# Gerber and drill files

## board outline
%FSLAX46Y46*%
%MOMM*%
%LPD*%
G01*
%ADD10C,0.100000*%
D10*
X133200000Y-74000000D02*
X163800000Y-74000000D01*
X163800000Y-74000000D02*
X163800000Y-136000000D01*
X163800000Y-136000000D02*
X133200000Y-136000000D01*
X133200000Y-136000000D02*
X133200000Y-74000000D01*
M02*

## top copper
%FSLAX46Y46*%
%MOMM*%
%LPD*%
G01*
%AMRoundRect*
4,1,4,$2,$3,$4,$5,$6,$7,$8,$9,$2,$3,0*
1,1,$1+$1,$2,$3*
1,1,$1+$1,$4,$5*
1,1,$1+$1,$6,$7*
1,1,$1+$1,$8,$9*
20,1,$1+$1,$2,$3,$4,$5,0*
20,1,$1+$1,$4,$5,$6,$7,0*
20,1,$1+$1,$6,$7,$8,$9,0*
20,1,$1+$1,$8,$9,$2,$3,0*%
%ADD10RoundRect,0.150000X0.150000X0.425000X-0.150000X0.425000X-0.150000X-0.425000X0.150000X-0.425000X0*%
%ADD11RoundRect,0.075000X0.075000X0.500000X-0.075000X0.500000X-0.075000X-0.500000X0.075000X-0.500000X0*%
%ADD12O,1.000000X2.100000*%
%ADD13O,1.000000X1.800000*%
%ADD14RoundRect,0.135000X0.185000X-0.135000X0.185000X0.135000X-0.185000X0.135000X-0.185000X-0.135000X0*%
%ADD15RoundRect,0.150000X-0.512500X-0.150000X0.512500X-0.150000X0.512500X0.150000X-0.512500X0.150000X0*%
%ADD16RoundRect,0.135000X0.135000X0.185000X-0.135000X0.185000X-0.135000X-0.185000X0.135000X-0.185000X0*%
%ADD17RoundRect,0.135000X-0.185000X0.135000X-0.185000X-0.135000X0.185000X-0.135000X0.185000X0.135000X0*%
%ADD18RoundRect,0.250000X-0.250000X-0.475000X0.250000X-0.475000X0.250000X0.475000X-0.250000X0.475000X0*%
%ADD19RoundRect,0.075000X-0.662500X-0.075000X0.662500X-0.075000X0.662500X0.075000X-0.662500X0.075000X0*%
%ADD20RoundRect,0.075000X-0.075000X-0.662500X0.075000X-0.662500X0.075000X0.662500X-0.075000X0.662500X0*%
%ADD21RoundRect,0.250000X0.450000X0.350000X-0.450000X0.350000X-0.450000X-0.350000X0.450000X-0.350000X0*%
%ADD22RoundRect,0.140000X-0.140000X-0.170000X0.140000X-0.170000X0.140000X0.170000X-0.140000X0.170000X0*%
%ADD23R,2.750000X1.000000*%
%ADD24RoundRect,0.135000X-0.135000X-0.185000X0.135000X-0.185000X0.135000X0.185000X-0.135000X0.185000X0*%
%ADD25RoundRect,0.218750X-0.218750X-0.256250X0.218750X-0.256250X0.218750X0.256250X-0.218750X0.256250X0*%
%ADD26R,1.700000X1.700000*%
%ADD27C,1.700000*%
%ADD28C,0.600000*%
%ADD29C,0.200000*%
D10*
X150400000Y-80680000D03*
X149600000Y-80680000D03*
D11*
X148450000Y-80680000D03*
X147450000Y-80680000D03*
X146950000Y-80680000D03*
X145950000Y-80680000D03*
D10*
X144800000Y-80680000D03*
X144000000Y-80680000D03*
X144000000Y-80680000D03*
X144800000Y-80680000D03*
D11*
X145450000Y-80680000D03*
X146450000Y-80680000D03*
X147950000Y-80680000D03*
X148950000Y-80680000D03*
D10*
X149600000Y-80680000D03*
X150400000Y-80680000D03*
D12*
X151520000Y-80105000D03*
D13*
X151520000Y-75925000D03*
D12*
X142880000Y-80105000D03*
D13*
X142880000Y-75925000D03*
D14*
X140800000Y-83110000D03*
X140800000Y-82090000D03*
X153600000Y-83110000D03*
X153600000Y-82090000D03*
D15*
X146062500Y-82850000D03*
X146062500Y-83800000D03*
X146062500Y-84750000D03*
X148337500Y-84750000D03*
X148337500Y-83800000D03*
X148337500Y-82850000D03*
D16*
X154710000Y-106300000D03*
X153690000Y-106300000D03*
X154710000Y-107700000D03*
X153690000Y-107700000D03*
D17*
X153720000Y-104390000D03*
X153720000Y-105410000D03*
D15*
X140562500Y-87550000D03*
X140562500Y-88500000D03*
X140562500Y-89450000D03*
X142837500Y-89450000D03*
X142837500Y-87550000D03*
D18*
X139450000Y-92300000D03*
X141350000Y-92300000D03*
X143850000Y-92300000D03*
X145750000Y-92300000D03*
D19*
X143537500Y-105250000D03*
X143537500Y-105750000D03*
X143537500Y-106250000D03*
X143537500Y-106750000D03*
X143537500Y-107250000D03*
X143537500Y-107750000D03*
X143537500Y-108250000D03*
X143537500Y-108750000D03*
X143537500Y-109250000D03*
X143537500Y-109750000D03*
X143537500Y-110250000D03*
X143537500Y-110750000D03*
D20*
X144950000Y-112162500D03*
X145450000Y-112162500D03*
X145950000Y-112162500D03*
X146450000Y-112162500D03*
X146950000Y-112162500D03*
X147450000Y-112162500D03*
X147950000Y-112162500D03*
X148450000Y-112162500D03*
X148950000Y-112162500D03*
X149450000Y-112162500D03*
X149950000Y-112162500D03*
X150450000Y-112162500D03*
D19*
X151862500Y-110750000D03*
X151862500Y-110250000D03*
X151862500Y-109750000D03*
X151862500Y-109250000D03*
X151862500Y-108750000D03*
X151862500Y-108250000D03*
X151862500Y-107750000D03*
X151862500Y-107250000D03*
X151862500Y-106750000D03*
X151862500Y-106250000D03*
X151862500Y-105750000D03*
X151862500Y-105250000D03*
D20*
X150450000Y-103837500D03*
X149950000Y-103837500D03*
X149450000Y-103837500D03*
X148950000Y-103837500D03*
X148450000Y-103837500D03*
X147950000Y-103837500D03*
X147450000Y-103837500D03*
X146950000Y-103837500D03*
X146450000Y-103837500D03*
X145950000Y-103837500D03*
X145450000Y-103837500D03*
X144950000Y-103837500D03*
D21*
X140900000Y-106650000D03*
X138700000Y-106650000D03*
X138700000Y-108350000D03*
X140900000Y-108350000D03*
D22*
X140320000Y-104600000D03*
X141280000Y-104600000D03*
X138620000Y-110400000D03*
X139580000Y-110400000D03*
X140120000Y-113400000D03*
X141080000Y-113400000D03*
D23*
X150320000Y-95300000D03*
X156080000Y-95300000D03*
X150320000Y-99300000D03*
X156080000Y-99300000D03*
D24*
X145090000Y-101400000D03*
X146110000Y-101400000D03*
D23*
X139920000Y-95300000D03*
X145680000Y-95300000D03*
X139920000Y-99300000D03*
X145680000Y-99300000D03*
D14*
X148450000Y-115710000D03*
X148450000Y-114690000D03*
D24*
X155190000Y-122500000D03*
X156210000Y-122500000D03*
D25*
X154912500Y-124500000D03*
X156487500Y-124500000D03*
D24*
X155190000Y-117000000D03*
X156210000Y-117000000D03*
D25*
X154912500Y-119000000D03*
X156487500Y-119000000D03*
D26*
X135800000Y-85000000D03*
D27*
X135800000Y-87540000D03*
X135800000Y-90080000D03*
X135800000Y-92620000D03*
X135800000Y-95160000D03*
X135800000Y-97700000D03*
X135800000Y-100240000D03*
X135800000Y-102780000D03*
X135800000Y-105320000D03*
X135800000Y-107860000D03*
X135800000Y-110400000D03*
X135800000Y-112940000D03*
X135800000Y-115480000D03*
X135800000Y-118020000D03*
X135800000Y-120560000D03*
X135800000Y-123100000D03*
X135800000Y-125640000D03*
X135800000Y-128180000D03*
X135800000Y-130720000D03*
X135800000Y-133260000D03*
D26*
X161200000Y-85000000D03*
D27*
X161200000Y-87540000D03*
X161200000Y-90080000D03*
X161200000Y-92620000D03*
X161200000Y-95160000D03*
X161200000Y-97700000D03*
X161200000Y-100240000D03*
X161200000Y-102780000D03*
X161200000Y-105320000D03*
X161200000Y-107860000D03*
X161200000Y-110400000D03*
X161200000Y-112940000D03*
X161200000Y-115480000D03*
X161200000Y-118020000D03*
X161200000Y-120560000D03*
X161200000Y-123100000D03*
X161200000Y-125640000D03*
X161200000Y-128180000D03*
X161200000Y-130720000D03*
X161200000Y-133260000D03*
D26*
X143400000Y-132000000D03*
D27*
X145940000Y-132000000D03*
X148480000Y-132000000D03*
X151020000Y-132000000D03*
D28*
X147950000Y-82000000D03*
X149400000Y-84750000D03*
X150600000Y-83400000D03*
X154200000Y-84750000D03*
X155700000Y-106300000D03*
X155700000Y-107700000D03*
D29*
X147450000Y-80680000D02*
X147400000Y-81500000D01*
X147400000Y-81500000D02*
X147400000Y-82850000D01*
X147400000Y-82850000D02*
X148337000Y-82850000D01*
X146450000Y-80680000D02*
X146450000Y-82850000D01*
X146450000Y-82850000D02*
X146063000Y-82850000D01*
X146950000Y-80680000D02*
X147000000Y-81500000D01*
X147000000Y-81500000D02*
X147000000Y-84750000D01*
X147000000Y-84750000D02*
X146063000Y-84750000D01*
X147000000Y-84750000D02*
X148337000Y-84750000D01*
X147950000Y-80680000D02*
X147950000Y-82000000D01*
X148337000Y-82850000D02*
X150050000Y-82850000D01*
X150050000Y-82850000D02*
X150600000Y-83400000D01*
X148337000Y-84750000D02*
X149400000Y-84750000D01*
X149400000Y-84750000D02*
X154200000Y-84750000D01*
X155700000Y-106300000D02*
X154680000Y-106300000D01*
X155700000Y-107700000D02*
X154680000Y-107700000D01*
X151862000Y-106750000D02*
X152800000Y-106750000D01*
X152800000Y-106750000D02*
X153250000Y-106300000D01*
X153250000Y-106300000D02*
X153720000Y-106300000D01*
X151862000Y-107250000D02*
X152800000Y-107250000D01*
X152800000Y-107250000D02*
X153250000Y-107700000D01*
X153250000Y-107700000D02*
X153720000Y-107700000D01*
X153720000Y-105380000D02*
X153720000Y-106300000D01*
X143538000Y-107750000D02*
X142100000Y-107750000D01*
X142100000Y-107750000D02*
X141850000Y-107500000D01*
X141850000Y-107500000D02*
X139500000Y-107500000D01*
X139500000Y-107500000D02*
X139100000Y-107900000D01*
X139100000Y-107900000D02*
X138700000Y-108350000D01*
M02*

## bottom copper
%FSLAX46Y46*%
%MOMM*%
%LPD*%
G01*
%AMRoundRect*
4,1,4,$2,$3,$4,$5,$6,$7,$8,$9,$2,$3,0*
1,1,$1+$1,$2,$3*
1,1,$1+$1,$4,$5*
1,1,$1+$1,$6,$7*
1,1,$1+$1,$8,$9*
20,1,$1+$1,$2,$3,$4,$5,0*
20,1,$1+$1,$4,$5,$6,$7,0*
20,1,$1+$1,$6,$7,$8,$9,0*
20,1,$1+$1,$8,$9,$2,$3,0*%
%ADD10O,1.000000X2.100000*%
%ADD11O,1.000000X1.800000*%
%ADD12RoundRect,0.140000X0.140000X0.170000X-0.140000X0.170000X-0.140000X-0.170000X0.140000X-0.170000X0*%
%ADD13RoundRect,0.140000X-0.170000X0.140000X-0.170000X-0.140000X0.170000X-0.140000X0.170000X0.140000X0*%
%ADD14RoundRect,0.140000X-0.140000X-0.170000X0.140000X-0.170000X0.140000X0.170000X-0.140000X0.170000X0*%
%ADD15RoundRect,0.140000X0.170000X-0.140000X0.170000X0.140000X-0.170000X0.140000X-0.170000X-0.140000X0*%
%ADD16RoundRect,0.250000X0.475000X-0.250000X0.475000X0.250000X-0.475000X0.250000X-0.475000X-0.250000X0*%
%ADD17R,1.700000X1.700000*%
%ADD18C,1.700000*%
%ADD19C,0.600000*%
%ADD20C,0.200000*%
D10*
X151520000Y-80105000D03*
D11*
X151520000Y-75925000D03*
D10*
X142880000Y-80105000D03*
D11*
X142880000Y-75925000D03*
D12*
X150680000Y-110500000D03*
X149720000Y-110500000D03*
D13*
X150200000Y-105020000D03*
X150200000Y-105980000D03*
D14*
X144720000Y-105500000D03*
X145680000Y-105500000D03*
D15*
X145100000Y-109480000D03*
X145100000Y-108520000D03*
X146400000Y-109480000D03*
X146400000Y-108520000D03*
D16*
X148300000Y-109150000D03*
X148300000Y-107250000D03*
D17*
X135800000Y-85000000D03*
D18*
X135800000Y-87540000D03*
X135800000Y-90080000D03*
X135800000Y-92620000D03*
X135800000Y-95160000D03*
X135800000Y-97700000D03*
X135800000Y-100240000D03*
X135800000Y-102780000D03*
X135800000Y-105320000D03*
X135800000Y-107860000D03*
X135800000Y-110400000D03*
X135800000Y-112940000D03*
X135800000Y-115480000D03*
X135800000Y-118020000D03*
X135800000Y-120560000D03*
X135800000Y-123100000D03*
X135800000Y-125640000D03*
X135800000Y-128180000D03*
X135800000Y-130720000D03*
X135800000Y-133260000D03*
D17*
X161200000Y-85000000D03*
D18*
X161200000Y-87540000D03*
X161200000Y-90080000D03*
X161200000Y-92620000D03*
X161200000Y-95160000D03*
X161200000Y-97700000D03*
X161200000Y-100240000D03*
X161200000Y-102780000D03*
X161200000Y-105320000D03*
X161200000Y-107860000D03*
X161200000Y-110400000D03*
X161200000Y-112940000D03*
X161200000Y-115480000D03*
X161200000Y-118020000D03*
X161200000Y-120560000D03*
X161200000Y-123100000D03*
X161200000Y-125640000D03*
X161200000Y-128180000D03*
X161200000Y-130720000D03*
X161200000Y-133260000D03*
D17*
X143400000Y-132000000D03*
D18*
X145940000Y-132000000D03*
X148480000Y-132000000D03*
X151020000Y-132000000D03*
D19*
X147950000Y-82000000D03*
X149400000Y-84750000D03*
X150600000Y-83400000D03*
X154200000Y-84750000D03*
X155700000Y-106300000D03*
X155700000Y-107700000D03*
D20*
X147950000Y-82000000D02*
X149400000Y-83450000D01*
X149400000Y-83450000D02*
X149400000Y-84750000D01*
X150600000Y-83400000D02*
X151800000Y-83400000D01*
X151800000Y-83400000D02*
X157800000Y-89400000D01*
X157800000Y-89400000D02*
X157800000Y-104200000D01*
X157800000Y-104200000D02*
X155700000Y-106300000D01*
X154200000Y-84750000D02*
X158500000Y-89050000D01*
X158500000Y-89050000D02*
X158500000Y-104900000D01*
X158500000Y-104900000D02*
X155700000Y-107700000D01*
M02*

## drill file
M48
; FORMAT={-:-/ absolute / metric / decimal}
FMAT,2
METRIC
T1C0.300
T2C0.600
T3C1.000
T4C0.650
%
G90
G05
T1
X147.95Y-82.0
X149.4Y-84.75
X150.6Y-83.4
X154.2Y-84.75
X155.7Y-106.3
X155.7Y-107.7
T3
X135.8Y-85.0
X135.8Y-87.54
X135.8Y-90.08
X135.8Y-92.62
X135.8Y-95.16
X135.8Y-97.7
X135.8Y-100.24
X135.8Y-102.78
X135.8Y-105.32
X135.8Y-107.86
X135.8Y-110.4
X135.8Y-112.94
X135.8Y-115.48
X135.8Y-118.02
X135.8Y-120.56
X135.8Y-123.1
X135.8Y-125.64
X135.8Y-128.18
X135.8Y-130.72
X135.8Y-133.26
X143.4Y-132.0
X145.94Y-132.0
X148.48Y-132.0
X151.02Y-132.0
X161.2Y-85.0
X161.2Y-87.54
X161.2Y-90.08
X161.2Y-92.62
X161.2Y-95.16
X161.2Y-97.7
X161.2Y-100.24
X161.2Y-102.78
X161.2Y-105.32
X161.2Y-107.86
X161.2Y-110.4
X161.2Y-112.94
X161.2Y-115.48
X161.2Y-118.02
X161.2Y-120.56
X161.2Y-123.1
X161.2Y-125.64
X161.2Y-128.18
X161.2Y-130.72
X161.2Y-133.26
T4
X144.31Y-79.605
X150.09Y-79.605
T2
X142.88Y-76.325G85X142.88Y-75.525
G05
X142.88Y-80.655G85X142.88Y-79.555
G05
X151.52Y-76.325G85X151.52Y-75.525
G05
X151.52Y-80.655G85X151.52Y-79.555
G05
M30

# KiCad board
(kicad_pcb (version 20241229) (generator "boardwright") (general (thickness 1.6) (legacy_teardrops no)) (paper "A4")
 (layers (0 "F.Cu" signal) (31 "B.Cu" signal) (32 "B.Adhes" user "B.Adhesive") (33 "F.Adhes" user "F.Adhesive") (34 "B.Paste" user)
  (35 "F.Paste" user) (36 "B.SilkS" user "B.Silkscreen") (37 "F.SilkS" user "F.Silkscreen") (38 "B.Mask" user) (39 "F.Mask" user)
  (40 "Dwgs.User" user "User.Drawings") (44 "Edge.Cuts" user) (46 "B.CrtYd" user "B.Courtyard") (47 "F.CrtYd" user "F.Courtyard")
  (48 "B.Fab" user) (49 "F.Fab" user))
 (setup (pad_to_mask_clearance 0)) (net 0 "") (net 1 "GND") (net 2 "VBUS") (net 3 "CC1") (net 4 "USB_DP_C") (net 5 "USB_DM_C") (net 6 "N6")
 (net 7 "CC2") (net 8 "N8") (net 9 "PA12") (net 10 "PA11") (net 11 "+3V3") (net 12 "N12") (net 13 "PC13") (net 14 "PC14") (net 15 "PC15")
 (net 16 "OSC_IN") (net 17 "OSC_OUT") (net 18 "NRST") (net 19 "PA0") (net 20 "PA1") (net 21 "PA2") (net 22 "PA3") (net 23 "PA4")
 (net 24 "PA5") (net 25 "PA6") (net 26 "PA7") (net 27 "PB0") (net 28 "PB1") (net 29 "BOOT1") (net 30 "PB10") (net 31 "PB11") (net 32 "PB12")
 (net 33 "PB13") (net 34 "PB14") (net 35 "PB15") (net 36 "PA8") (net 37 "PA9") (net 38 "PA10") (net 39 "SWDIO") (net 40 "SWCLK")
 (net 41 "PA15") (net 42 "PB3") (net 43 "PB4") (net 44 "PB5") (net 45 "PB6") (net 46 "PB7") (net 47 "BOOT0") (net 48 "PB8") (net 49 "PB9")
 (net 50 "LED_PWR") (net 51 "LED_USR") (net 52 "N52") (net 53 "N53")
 (gr_line (start 133.2 74) (end 163.8 74) (stroke (width 0.1) (type default)) (layer "Edge.Cuts"))
 (gr_line (start 163.8 74) (end 163.8 136) (stroke (width 0.1) (type default)) (layer "Edge.Cuts"))
 (gr_line (start 163.8 136) (end 133.2 136) (stroke (width 0.1) (type default)) (layer "Edge.Cuts"))
 (gr_line (start 133.2 136) (end 133.2 74) (stroke (width 0.1) (type default)) (layer "Edge.Cuts"))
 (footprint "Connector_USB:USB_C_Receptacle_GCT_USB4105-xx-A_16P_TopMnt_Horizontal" (layer "F.Cu") (at 147.2 77 180)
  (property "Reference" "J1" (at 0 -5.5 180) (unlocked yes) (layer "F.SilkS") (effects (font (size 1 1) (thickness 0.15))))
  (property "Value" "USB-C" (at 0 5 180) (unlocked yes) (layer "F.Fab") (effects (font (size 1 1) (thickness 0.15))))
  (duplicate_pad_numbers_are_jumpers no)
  (pad "" np_thru_hole circle (at -2.89 -2.605 180) (size 0.65 0.65) (drill 0.65) (layers "*.Cu" "*.Mask"))
  (pad "" np_thru_hole circle (at 2.89 -2.605 180) (size 0.65 0.65) (drill 0.65) (layers "*.Cu" "*.Mask"))
  (pad "A1" smd roundrect (at -3.2 -3.68 180) (size 0.6 1.15) (layers "F.Cu" "F.Mask" "F.Paste") (roundrect_rratio 0.25) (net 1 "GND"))
  (pad "A4" smd roundrect (at -2.4 -3.68 180) (size 0.6 1.15) (layers "F.Cu" "F.Mask" "F.Paste") (roundrect_rratio 0.25) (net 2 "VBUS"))
  (pad "A5" smd roundrect (at -1.25 -3.68 180) (size 0.3 1.15) (layers "F.Cu" "F.Mask" "F.Paste") (roundrect_rratio 0.25) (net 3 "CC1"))
  (pad "A6" smd roundrect (at -0.25 -3.68 180) (size 0.3 1.15) (layers "F.Cu" "F.Mask" "F.Paste") (roundrect_rratio 0.25) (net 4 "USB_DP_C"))
  (pad "A7" smd roundrect (at 0.25 -3.68 180) (size 0.3 1.15) (layers "F.Cu" "F.Mask" "F.Paste") (roundrect_rratio 0.25) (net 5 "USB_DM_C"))
  (pad "A8" smd roundrect (at 1.25 -3.68 180) (size 0.3 1.15) (layers "F.Cu" "F.Mask" "F.Paste") (roundrect_rratio 0.25) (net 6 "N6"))
  (pad "A9" smd roundrect (at 2.4 -3.68 180) (size 0.6 1.15) (layers "F.Cu" "F.Mask" "F.Paste") (roundrect_rratio 0.25) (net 2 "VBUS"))
  (pad "A12" smd roundrect (at 3.2 -3.68 180) (size 0.6 1.15) (layers "F.Cu" "F.Mask" "F.Paste") (roundrect_rratio 0.25) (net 1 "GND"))
  (pad "B1" smd roundrect (at 3.2 -3.68 180) (size 0.6 1.15) (layers "F.Cu" "F.Mask" "F.Paste") (roundrect_rratio 0.25) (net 1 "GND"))
  (pad "B4" smd roundrect (at 2.4 -3.68 180) (size 0.6 1.15) (layers "F.Cu" "F.Mask" "F.Paste") (roundrect_rratio 0.25) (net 2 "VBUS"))
  (pad "B5" smd roundrect (at 1.75 -3.68 180) (size 0.3 1.15) (layers "F.Cu" "F.Mask" "F.Paste") (roundrect_rratio 0.25) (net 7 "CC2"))
  (pad "B6" smd roundrect (at 0.75 -3.68 180) (size 0.3 1.15) (layers "F.Cu" "F.Mask" "F.Paste") (roundrect_rratio 0.25) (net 4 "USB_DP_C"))
  (pad "B7" smd roundrect (at -0.75 -3.68 180) (size 0.3 1.15) (layers "F.Cu" "F.Mask" "F.Paste") (roundrect_rratio 0.25) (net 5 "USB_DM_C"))
  (pad "B8" smd roundrect (at -1.75 -3.68 180) (size 0.3 1.15) (layers "F.Cu" "F.Mask" "F.Paste") (roundrect_rratio 0.25) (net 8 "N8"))
  (pad "B9" smd roundrect (at -2.4 -3.68 180) (size 0.6 1.15) (layers "F.Cu" "F.Mask" "F.Paste") (roundrect_rratio 0.25) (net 2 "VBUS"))
  (pad "B12" smd roundrect (at -3.2 -3.68 180) (size 0.6 1.15) (layers "F.Cu" "F.Mask" "F.Paste") (roundrect_rratio 0.25) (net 1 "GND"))
  (pad "SH" thru_hole oval (at -4.32 -3.105 180) (size 1 2.1) (drill oval 0.6 1.7) (layers "*.Cu" "*.Mask" "F.Paste")
   (remove_unused_layers no) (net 1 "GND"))
  (pad "SH" thru_hole oval (at -4.32 1.075 180) (size 1 1.8) (drill oval 0.6 1.4) (layers "*.Cu" "*.Mask" "F.Paste")
   (remove_unused_layers no) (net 1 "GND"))
  (pad "SH" thru_hole oval (at 4.32 -3.105 180) (size 1 2.1) (drill oval 0.6 1.7) (layers "*.Cu" "*.Mask" "F.Paste")
   (remove_unused_layers no) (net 1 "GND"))
  (pad "SH" thru_hole oval (at 4.32 1.075 180) (size 1 1.8) (drill oval 0.6 1.4) (layers "*.Cu" "*.Mask" "F.Paste")
   (remove_unused_layers no) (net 1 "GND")))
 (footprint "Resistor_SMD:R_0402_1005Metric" (layer "F.Cu") (at 140.8 82.6 90)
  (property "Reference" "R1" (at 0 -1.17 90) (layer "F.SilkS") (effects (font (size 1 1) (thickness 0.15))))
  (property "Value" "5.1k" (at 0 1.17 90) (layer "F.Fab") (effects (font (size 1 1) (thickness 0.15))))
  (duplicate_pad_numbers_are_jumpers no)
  (pad "1" smd roundrect (at -0.51 0 90) (size 0.54 0.64) (layers "F.Cu" "F.Mask" "F.Paste") (roundrect_rratio 0.25) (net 3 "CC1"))
  (pad "2" smd roundrect (at 0.51 0 90) (size 0.54 0.64) (layers "F.Cu" "F.Mask" "F.Paste") (roundrect_rratio 0.25) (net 1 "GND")))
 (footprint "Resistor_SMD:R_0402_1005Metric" (layer "F.Cu") (at 153.6 82.6 90)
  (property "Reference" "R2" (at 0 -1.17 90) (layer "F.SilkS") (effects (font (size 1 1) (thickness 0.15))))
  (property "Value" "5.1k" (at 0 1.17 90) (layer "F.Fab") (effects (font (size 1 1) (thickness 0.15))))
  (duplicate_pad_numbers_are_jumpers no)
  (pad "1" smd roundrect (at -0.51 0 90) (size 0.54 0.64) (layers "F.Cu" "F.Mask" "F.Paste") (roundrect_rratio 0.25) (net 7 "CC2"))
  (pad "2" smd roundrect (at 0.51 0 90) (size 0.54 0.64) (layers "F.Cu" "F.Mask" "F.Paste") (roundrect_rratio 0.25) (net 1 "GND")))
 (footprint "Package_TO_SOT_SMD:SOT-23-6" (layer "F.Cu") (at 147.2 83.8)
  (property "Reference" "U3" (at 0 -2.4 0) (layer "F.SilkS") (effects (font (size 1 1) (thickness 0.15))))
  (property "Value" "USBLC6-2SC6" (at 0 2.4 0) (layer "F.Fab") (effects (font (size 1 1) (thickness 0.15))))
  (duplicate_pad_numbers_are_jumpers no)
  (pad "1" smd roundrect (at -1.1375 -0.95) (size 1.325 0.6) (layers "F.Cu" "F.Mask" "F.Paste") (roundrect_rratio 0.25) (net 4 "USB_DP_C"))
  (pad "2" smd roundrect (at -1.1375 0) (size 1.325 0.6) (layers "F.Cu" "F.Mask" "F.Paste") (roundrect_rratio 0.25) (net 1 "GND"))
  (pad "3" smd roundrect (at -1.1375 0.95) (size 1.325 0.6) (layers "F.Cu" "F.Mask" "F.Paste") (roundrect_rratio 0.25) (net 5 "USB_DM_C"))
  (pad "4" smd roundrect (at 1.1375 0.95) (size 1.325 0.6) (layers "F.Cu" "F.Mask" "F.Paste") (roundrect_rratio 0.25) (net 5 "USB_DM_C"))
  (pad "5" smd roundrect (at 1.1375 0) (size 1.325 0.6) (layers "F.Cu" "F.Mask" "F.Paste") (roundrect_rratio 0.25) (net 2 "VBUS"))
  (pad "6" smd roundrect (at 1.1375 -0.95) (size 1.325 0.6) (layers "F.Cu" "F.Mask" "F.Paste") (roundrect_rratio 0.25) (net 4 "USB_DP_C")))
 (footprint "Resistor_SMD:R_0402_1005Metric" (layer "F.Cu") (at 154.2 106.3 180)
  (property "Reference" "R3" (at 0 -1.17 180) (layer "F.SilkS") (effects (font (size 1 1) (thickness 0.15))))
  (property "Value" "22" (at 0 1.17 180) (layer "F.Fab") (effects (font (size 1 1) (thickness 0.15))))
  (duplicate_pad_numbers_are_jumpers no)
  (pad "1" smd roundrect (at -0.51 0 180) (size 0.54 0.64) (layers "F.Cu" "F.Mask" "F.Paste") (roundrect_rratio 0.25) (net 4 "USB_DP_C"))
  (pad "2" smd roundrect (at 0.51 0 180) (size 0.54 0.64) (layers "F.Cu" "F.Mask" "F.Paste") (roundrect_rratio 0.25) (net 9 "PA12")))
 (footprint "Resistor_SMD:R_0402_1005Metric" (layer "F.Cu") (at 154.2 107.7 180)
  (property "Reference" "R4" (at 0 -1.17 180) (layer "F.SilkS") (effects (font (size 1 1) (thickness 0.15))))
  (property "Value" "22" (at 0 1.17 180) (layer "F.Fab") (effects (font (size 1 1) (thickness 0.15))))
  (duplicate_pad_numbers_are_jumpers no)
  (pad "1" smd roundrect (at -0.51 0 180) (size 0.54 0.64) (layers "F.Cu" "F.Mask" "F.Paste") (roundrect_rratio 0.25) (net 5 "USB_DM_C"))
  (pad "2" smd roundrect (at 0.51 0 180) (size 0.54 0.64) (layers "F.Cu" "F.Mask" "F.Paste") (roundrect_rratio 0.25) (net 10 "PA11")))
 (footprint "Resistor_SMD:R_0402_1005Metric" (layer "F.Cu") (at 153.72 104.9 -90)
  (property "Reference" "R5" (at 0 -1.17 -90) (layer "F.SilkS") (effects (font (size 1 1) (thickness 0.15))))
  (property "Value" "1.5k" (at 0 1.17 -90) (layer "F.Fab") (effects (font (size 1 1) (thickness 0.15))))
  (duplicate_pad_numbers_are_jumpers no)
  (pad "1" smd roundrect (at -0.51 0 -90) (size 0.54 0.64) (layers "F.Cu" "F.Mask" "F.Paste") (roundrect_rratio 0.25) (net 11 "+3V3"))
  (pad "2" smd roundrect (at 0.51 0 -90) (size 0.54 0.64) (layers "F.Cu" "F.Mask" "F.Paste") (roundrect_rratio 0.25) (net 9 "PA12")))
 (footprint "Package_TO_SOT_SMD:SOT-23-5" (layer "F.Cu") (at 141.7 88.5)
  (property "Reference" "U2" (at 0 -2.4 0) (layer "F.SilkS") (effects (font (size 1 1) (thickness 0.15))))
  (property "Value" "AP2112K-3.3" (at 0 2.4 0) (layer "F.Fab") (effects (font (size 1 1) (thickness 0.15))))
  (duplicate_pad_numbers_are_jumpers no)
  (pad "1" smd roundrect (at -1.1375 -0.95) (size 1.325 0.6) (layers "F.Cu" "F.Mask" "F.Paste") (roundrect_rratio 0.25) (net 2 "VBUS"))
  (pad "2" smd roundrect (at -1.1375 0) (size 1.325 0.6) (layers "F.Cu" "F.Mask" "F.Paste") (roundrect_rratio 0.25) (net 1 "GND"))
  (pad "3" smd roundrect (at -1.1375 0.95) (size 1.325 0.6) (layers "F.Cu" "F.Mask" "F.Paste") (roundrect_rratio 0.25) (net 2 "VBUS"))
  (pad "4" smd roundrect (at 1.1375 0.95) (size 1.325 0.6) (layers "F.Cu" "F.Mask" "F.Paste") (roundrect_rratio 0.25) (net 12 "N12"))
  (pad "5" smd roundrect (at 1.1375 -0.95) (size 1.325 0.6) (layers "F.Cu" "F.Mask" "F.Paste") (roundrect_rratio 0.25) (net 11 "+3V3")))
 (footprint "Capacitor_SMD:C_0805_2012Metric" (layer "F.Cu") (at 140.4 92.3)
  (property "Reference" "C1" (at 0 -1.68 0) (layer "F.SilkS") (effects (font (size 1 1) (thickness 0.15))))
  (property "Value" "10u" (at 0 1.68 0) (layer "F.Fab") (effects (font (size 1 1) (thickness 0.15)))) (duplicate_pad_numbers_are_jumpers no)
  (pad "1" smd roundrect (at -0.95 0) (size 1 1.45) (layers "F.Cu" "F.Mask" "F.Paste") (roundrect_rratio 0.25) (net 2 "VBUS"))
  (pad "2" smd roundrect (at 0.95 0) (size 1 1.45) (layers "F.Cu" "F.Mask" "F.Paste") (roundrect_rratio 0.25) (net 1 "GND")))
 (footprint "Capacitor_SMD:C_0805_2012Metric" (layer "F.Cu") (at 144.8 92.3)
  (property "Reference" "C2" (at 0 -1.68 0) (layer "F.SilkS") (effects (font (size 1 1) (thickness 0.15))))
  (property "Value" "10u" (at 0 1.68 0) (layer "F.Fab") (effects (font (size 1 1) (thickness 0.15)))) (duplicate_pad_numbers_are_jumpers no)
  (pad "1" smd roundrect (at -0.95 0) (size 1 1.45) (layers "F.Cu" "F.Mask" "F.Paste") (roundrect_rratio 0.25) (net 11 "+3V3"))
  (pad "2" smd roundrect (at 0.95 0) (size 1 1.45) (layers "F.Cu" "F.Mask" "F.Paste") (roundrect_rratio 0.25) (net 1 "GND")))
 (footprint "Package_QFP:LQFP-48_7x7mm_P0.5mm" (layer "F.Cu") (at 147.7 108)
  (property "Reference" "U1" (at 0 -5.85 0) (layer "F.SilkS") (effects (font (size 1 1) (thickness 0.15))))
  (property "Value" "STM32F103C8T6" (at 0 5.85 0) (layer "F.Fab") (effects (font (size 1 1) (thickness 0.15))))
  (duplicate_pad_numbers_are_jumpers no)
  (pad "1" smd roundrect (at -4.1625 -2.75) (size 1.475 0.3) (layers "F.Cu" "F.Mask" "F.Paste") (roundrect_rratio 0.25) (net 11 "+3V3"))
  (pad "2" smd roundrect (at -4.1625 -2.25) (size 1.475 0.3) (layers "F.Cu" "F.Mask" "F.Paste") (roundrect_rratio 0.25) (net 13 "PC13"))
  (pad "3" smd roundrect (at -4.1625 -1.75) (size 1.475 0.3) (layers "F.Cu" "F.Mask" "F.Paste") (roundrect_rratio 0.25) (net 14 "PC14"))
  (pad "4" smd roundrect (at -4.1625 -1.25) (size 1.475 0.3) (layers "F.Cu" "F.Mask" "F.Paste") (roundrect_rratio 0.25) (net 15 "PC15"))
  (pad "5" smd roundrect (at -4.1625 -0.75) (size 1.475 0.3) (layers "F.Cu" "F.Mask" "F.Paste") (roundrect_rratio 0.25) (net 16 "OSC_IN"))
  (pad "6" smd roundrect (at -4.1625 -0.25) (size 1.475 0.3) (layers "F.Cu" "F.Mask" "F.Paste") (roundrect_rratio 0.25) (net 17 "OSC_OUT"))
  (pad "7" smd roundrect (at -4.1625 0.25) (size 1.475 0.3) (layers "F.Cu" "F.Mask" "F.Paste") (roundrect_rratio 0.25) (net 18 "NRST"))
  (pad "8" smd roundrect (at -4.1625 0.75) (size 1.475 0.3) (layers "F.Cu" "F.Mask" "F.Paste") (roundrect_rratio 0.25) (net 1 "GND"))
  (pad "9" smd roundrect (at -4.1625 1.25) (size 1.475 0.3) (layers "F.Cu" "F.Mask" "F.Paste") (roundrect_rratio 0.25) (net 11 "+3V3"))
  (pad "10" smd roundrect (at -4.1625 1.75) (size 1.475 0.3) (layers "F.Cu" "F.Mask" "F.Paste") (roundrect_rratio 0.25) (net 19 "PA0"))
  (pad "11" smd roundrect (at -4.1625 2.25) (size 1.475 0.3) (layers "F.Cu" "F.Mask" "F.Paste") (roundrect_rratio 0.25) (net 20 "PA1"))
  (pad "12" smd roundrect (at -4.1625 2.75) (size 1.475 0.3) (layers "F.Cu" "F.Mask" "F.Paste") (roundrect_rratio 0.25) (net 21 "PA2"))
  (pad "13" smd roundrect (at -2.75 4.1625) (size 0.3 1.475) (layers "F.Cu" "F.Mask" "F.Paste") (roundrect_rratio 0.25) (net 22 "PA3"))
  (pad "14" smd roundrect (at -2.25 4.1625) (size 0.3 1.475) (layers "F.Cu" "F.Mask" "F.Paste") (roundrect_rratio 0.25) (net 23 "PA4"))
  (pad "15" smd roundrect (at -1.75 4.1625) (size 0.3 1.475) (layers "F.Cu" "F.Mask" "F.Paste") (roundrect_rratio 0.25) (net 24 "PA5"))
  (pad "16" smd roundrect (at -1.25 4.1625) (size 0.3 1.475) (layers "F.Cu" "F.Mask" "F.Paste") (roundrect_rratio 0.25) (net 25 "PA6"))
  (pad "17" smd roundrect (at -0.75 4.1625) (size 0.3 1.475) (layers "F.Cu" "F.Mask" "F.Paste") (roundrect_rratio 0.25) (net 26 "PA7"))
  (pad "18" smd roundrect (at -0.25 4.1625) (size 0.3 1.475) (layers "F.Cu" "F.Mask" "F.Paste") (roundrect_rratio 0.25) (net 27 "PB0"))
  (pad "19" smd roundrect (at 0.25 4.1625) (size 0.3 1.475) (layers "F.Cu" "F.Mask" "F.Paste") (roundrect_rratio 0.25) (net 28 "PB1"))
  (pad "20" smd roundrect (at 0.75 4.1625) (size 0.3 1.475) (layers "F.Cu" "F.Mask" "F.Paste") (roundrect_rratio 0.25) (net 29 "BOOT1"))
  (pad "21" smd roundrect (at 1.25 4.1625) (size 0.3 1.475) (layers "F.Cu" "F.Mask" "F.Paste") (roundrect_rratio 0.25) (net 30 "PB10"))
  (pad "22" smd roundrect (at 1.75 4.1625) (size 0.3 1.475) (layers "F.Cu" "F.Mask" "F.Paste") (roundrect_rratio 0.25) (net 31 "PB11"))
  (pad "23" smd roundrect (at 2.25 4.1625) (size 0.3 1.475) (layers "F.Cu" "F.Mask" "F.Paste") (roundrect_rratio 0.25) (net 1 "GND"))
  (pad "24" smd roundrect (at 2.75 4.1625) (size 0.3 1.475) (layers "F.Cu" "F.Mask" "F.Paste") (roundrect_rratio 0.25) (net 11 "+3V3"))
  (pad "25" smd roundrect (at 4.1625 2.75) (size 1.475 0.3) (layers "F.Cu" "F.Mask" "F.Paste") (roundrect_rratio 0.25) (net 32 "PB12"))
  (pad "26" smd roundrect (at 4.1625 2.25) (size 1.475 0.3) (layers "F.Cu" "F.Mask" "F.Paste") (roundrect_rratio 0.25) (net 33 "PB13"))
  (pad "27" smd roundrect (at 4.1625 1.75) (size 1.475 0.3) (layers "F.Cu" "F.Mask" "F.Paste") (roundrect_rratio 0.25) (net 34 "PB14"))
  (pad "28" smd roundrect (at 4.1625 1.25) (size 1.475 0.3) (layers "F.Cu" "F.Mask" "F.Paste") (roundrect_rratio 0.25) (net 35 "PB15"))
  (pad "29" smd roundrect (at 4.1625 0.75) (size 1.475 0.3) (layers "F.Cu" "F.Mask" "F.Paste") (roundrect_rratio 0.25) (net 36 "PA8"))
  (pad "30" smd roundrect (at 4.1625 0.25) (size 1.475 0.3) (layers "F.Cu" "F.Mask" "F.Paste") (roundrect_rratio 0.25) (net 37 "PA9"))
  (pad "31" smd roundrect (at 4.1625 -0.25) (size 1.475 0.3) (layers "F.Cu" "F.Mask" "F.Paste") (roundrect_rratio 0.25) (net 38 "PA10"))
  (pad "32" smd roundrect (at 4.1625 -0.75) (size 1.475 0.3) (layers "F.Cu" "F.Mask" "F.Paste") (roundrect_rratio 0.25) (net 10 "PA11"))
  (pad "33" smd roundrect (at 4.1625 -1.25) (size 1.475 0.3) (layers "F.Cu" "F.Mask" "F.Paste") (roundrect_rratio 0.25) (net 9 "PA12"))
  (pad "34" smd roundrect (at 4.1625 -1.75) (size 1.475 0.3) (layers "F.Cu" "F.Mask" "F.Paste") (roundrect_rratio 0.25) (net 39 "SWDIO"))
  (pad "35" smd roundrect (at 4.1625 -2.25) (size 1.475 0.3) (layers "F.Cu" "F.Mask" "F.Paste") (roundrect_rratio 0.25) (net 1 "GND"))
  (pad "36" smd roundrect (at 4.1625 -2.75) (size 1.475 0.3) (layers "F.Cu" "F.Mask" "F.Paste") (roundrect_rratio 0.25) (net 11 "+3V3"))
  (pad "37" smd roundrect (at 2.75 -4.1625) (size 0.3 1.475) (layers "F.Cu" "F.Mask" "F.Paste") (roundrect_rratio 0.25) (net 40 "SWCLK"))
  (pad "38" smd roundrect (at 2.25 -4.1625) (size 0.3 1.475) (layers "F.Cu" "F.Mask" "F.Paste") (roundrect_rratio 0.25) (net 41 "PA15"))
  (pad "39" smd roundrect (at 1.75 -4.1625) (size 0.3 1.475) (layers "F.Cu" "F.Mask" "F.Paste") (roundrect_rratio 0.25) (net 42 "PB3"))
  (pad "40" smd roundrect (at 1.25 -4.1625) (size 0.3 1.475) (layers "F.Cu" "F.Mask" "F.Paste") (roundrect_rratio 0.25) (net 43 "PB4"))
  (pad "41" smd roundrect (at 0.75 -4.1625) (size 0.3 1.475) (layers "F.Cu" "F.Mask" "F.Paste") (roundrect_rratio 0.25) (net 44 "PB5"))
  (pad "42" smd roundrect (at 0.25 -4.1625) (size 0.3 1.475) (layers "F.Cu" "F.Mask" "F.Paste") (roundrect_rratio 0.25) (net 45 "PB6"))
  (pad "43" smd roundrect (at -0.25 -4.1625) (size 0.3 1.475) (layers "F.Cu" "F.Mask" "F.Paste") (roundrect_rratio 0.25) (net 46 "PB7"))
  (pad "44" smd roundrect (at -0.75 -4.1625) (size 0.3 1.475) (layers "F.Cu" "F.Mask" "F.Paste") (roundrect_rratio 0.25) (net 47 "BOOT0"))
  (pad "45" smd roundrect (at -1.25 -4.1625) (size 0.3 1.475) (layers "F.Cu" "F.Mask" "F.Paste") (roundrect_rratio 0.25) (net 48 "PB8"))
  (pad "46" smd roundrect (at -1.75 -4.1625) (size 0.3 1.475) (layers "F.Cu" "F.Mask" "F.Paste") (roundrect_rratio 0.25) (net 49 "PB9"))
  (pad "47" smd roundrect (at -2.25 -4.1625) (size 0.3 1.475) (layers "F.Cu" "F.Mask" "F.Paste") (roundrect_rratio 0.25) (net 1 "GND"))
  (pad "48" smd roundrect (at -2.75 -4.1625) (size 0.3 1.475) (layers "F.Cu" "F.Mask" "F.Paste") (roundrect_rratio 0.25) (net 11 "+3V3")))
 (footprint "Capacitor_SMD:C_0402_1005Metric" (layer "B.Cu") (at 150.2 110.5 180)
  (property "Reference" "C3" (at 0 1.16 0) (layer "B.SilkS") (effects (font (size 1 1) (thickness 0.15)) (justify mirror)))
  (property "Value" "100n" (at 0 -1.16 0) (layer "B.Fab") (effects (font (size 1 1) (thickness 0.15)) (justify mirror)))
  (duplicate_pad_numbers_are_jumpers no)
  (pad "1" smd roundrect (at -0.48 0 180) (size 0.56 0.62) (layers "B.Cu" "B.Mask" "B.Paste") (roundrect_rratio 0.25) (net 11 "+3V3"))
  (pad "2" smd roundrect (at 0.48 0 180) (size 0.56 0.62) (layers "B.Cu" "B.Mask" "B.Paste") (roundrect_rratio 0.25) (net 1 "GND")))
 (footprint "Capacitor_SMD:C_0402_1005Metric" (layer "B.Cu") (at 150.2 105.5 -90)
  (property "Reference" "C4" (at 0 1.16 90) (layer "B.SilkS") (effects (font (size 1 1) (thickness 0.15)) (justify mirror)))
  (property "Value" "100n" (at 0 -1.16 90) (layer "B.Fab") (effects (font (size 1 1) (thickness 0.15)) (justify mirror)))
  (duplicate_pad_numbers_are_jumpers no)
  (pad "1" smd roundrect (at -0.48 0 -90) (size 0.56 0.62) (layers "B.Cu" "B.Mask" "B.Paste") (roundrect_rratio 0.25) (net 11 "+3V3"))
  (pad "2" smd roundrect (at 0.48 0 -90) (size 0.56 0.62) (layers "B.Cu" "B.Mask" "B.Paste") (roundrect_rratio 0.25) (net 1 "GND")))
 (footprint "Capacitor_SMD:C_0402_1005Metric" (layer "B.Cu") (at 145.2 105.5)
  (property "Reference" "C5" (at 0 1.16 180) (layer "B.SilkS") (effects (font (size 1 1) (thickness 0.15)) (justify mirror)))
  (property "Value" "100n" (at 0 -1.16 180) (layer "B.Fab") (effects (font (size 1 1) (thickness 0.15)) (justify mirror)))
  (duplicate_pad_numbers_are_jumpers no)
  (pad "1" smd roundrect (at -0.48 0) (size 0.56 0.62) (layers "B.Cu" "B.Mask" "B.Paste") (roundrect_rratio 0.25) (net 11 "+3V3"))
  (pad "2" smd roundrect (at 0.48 0) (size 0.56 0.62) (layers "B.Cu" "B.Mask" "B.Paste") (roundrect_rratio 0.25) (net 1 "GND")))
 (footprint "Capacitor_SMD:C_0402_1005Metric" (layer "B.Cu") (at 145.1 109 90)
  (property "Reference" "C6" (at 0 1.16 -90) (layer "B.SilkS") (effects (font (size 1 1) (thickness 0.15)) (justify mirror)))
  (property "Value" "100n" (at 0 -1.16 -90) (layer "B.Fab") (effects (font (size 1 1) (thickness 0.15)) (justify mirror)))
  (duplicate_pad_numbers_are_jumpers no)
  (pad "1" smd roundrect (at -0.48 0 90) (size 0.56 0.62) (layers "B.Cu" "B.Mask" "B.Paste") (roundrect_rratio 0.25) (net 11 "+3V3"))
  (pad "2" smd roundrect (at 0.48 0 90) (size 0.56 0.62) (layers "B.Cu" "B.Mask" "B.Paste") (roundrect_rratio 0.25) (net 1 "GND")))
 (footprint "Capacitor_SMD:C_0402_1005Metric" (layer "B.Cu") (at 146.4 109 90)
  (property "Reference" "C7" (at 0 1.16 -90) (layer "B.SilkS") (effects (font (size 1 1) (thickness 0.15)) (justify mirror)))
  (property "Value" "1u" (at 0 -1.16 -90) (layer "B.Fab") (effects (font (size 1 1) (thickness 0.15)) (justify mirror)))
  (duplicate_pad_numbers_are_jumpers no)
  (pad "1" smd roundrect (at -0.48 0 90) (size 0.56 0.62) (layers "B.Cu" "B.Mask" "B.Paste") (roundrect_rratio 0.25) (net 11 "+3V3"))
  (pad "2" smd roundrect (at 0.48 0 90) (size 0.56 0.62) (layers "B.Cu" "B.Mask" "B.Paste") (roundrect_rratio 0.25) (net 1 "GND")))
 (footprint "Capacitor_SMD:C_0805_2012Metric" (layer "B.Cu") (at 148.3 108.2 90)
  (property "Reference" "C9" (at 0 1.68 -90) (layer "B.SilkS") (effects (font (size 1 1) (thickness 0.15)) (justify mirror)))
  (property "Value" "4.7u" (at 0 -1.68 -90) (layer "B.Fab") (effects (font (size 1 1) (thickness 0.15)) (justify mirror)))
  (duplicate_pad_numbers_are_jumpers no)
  (pad "1" smd roundrect (at -0.95 0 90) (size 1 1.45) (layers "B.Cu" "B.Mask" "B.Paste") (roundrect_rratio 0.25) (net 11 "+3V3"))
  (pad "2" smd roundrect (at 0.95 0 90) (size 1 1.45) (layers "B.Cu" "B.Mask" "B.Paste") (roundrect_rratio 0.25) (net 1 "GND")))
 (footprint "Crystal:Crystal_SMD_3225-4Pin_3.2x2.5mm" (layer "F.Cu") (at 139.8 107.5 180)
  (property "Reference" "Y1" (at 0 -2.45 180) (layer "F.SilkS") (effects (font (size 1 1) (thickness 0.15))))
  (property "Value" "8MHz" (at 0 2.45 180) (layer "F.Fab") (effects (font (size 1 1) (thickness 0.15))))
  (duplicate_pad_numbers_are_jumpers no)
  (pad "1" smd roundrect (at -1.1 0.85 180) (size 1.4 1.2) (layers "F.Cu" "F.Mask" "F.Paste") (roundrect_rratio 0.208333) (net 16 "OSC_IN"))
  (pad "2" smd roundrect (at 1.1 0.85 180) (size 1.4 1.2) (layers "F.Cu" "F.Mask" "F.Paste") (roundrect_rratio 0.208333) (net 1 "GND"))
  (pad "3" smd roundrect (at 1.1 -0.85 180) (size 1.4 1.2) (layers "F.Cu" "F.Mask" "F.Paste") (roundrect_rratio 0.208333) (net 17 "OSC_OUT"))
  (pad "4" smd roundrect (at -1.1 -0.85 180) (size 1.4 1.2) (layers "F.Cu" "F.Mask" "F.Paste") (roundrect_rratio 0.208333) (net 1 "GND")))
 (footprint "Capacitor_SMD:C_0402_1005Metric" (layer "F.Cu") (at 140.8 104.6)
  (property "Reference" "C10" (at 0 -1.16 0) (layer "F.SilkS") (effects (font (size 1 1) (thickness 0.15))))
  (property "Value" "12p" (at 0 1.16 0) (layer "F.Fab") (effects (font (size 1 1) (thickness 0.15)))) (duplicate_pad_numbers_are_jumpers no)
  (pad "1" smd roundrect (at -0.48 0) (size 0.56 0.62) (layers "F.Cu" "F.Mask" "F.Paste") (roundrect_rratio 0.25) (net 16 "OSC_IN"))
  (pad "2" smd roundrect (at 0.48 0) (size 0.56 0.62) (layers "F.Cu" "F.Mask" "F.Paste") (roundrect_rratio 0.25) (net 1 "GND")))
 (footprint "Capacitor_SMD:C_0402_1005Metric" (layer "F.Cu") (at 139.1 110.4)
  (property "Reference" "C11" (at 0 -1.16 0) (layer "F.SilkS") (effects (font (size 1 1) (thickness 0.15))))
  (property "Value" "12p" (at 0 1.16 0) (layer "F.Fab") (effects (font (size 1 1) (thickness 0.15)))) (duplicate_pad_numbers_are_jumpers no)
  (pad "1" smd roundrect (at -0.48 0) (size 0.56 0.62) (layers "F.Cu" "F.Mask" "F.Paste") (roundrect_rratio 0.25) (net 17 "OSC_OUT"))
  (pad "2" smd roundrect (at 0.48 0) (size 0.56 0.62) (layers "F.Cu" "F.Mask" "F.Paste") (roundrect_rratio 0.25) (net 1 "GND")))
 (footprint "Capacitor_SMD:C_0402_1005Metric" (layer "F.Cu") (at 140.6 113.4)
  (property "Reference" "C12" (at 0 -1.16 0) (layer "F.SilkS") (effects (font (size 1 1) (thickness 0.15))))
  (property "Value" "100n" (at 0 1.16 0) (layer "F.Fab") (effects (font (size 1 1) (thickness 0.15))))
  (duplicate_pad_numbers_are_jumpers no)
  (pad "1" smd roundrect (at -0.48 0) (size 0.56 0.62) (layers "F.Cu" "F.Mask" "F.Paste") (roundrect_rratio 0.25) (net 18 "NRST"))
  (pad "2" smd roundrect (at 0.48 0) (size 0.56 0.62) (layers "F.Cu" "F.Mask" "F.Paste") (roundrect_rratio 0.25) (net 1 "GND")))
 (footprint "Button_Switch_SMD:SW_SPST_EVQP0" (layer "F.Cu") (at 153.2 97.3)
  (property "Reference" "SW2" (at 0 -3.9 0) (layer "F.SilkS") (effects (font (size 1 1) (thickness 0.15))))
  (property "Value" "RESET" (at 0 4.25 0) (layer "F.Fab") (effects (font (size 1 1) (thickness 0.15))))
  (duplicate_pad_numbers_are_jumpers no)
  (pad "1" smd rect (at -2.88 -2) (size 2.75 1) (layers "F.Cu" "F.Mask" "F.Paste") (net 18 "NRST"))
  (pad "1" smd rect (at 2.88 -2) (size 2.75 1) (layers "F.Cu" "F.Mask" "F.Paste") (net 18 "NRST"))
  (pad "2" smd rect (at -2.88 2) (size 2.75 1) (layers "F.Cu" "F.Mask" "F.Paste") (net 1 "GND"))
  (pad "2" smd rect (at 2.88 2) (size 2.75 1) (layers "F.Cu" "F.Mask" "F.Paste") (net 1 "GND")))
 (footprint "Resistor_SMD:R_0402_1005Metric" (layer "F.Cu") (at 145.6 101.4)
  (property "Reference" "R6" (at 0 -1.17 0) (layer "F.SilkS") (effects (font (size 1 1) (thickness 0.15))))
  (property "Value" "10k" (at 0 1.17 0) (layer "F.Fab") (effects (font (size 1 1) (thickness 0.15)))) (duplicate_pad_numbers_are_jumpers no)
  (pad "1" smd roundrect (at -0.51 0) (size 0.54 0.64) (layers "F.Cu" "F.Mask" "F.Paste") (roundrect_rratio 0.25) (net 47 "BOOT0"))
  (pad "2" smd roundrect (at 0.51 0) (size 0.54 0.64) (layers "F.Cu" "F.Mask" "F.Paste") (roundrect_rratio 0.25) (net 1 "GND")))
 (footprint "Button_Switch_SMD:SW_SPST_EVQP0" (layer "F.Cu") (at 142.8 97.3)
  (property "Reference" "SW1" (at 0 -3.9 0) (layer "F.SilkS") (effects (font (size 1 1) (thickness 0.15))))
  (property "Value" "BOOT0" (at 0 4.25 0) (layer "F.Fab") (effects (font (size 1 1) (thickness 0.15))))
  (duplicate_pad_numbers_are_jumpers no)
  (pad "1" smd rect (at -2.88 -2) (size 2.75 1) (layers "F.Cu" "F.Mask" "F.Paste") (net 47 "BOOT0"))
  (pad "1" smd rect (at 2.88 -2) (size 2.75 1) (layers "F.Cu" "F.Mask" "F.Paste") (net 47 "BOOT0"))
  (pad "2" smd rect (at -2.88 2) (size 2.75 1) (layers "F.Cu" "F.Mask" "F.Paste") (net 11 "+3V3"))
  (pad "2" smd rect (at 2.88 2) (size 2.75 1) (layers "F.Cu" "F.Mask" "F.Paste") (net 11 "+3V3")))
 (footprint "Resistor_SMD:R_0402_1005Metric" (layer "F.Cu") (at 148.45 115.2 90)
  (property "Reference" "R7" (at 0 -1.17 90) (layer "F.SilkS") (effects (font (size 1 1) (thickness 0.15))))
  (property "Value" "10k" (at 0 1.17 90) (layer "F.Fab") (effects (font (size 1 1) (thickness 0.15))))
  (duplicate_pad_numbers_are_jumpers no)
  (pad "1" smd roundrect (at -0.51 0 90) (size 0.54 0.64) (layers "F.Cu" "F.Mask" "F.Paste") (roundrect_rratio 0.25) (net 29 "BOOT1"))
  (pad "2" smd roundrect (at 0.51 0 90) (size 0.54 0.64) (layers "F.Cu" "F.Mask" "F.Paste") (roundrect_rratio 0.25) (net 1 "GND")))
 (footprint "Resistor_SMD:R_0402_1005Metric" (layer "F.Cu") (at 155.7 122.5)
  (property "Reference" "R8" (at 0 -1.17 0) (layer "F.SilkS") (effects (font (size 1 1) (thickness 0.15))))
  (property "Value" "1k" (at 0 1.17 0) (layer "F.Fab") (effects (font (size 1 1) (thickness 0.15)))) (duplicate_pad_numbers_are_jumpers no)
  (pad "1" smd roundrect (at -0.51 0) (size 0.54 0.64) (layers "F.Cu" "F.Mask" "F.Paste") (roundrect_rratio 0.25) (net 11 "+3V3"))
  (pad "2" smd roundrect (at 0.51 0) (size 0.54 0.64) (layers "F.Cu" "F.Mask" "F.Paste") (roundrect_rratio 0.25) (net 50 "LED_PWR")))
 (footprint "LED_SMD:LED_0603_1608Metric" (layer "F.Cu") (at 155.7 124.5)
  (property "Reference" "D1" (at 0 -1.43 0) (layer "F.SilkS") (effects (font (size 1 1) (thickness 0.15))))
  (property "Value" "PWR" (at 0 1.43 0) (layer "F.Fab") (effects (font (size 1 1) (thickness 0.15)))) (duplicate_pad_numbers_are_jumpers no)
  (pad "1" smd roundrect (at -0.7875 0) (size 0.875 0.95) (layers "F.Cu" "F.Mask" "F.Paste") (roundrect_rratio 0.25) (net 1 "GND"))
  (pad "2" smd roundrect (at 0.7875 0) (size 0.875 0.95) (layers "F.Cu" "F.Mask" "F.Paste") (roundrect_rratio 0.25) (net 50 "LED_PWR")))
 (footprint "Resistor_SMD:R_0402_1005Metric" (layer "F.Cu") (at 155.7 117)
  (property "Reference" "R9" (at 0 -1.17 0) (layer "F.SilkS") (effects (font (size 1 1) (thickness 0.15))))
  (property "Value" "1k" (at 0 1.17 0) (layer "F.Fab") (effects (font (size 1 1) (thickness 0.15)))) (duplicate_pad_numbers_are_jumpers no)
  (pad "1" smd roundrect (at -0.51 0) (size 0.54 0.64) (layers "F.Cu" "F.Mask" "F.Paste") (roundrect_rratio 0.25) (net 11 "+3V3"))
  (pad "2" smd roundrect (at 0.51 0) (size 0.54 0.64) (layers "F.Cu" "F.Mask" "F.Paste") (roundrect_rratio 0.25) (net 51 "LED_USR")))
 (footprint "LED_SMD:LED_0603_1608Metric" (layer "F.Cu") (at 155.7 119)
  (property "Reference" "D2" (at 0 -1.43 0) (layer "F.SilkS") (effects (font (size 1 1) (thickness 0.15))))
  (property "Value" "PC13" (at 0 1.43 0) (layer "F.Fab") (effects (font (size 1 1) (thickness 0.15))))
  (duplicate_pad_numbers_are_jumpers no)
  (pad "1" smd roundrect (at -0.7875 0) (size 0.875 0.95) (layers "F.Cu" "F.Mask" "F.Paste") (roundrect_rratio 0.25) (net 13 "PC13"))
  (pad "2" smd roundrect (at 0.7875 0) (size 0.875 0.95) (layers "F.Cu" "F.Mask" "F.Paste") (roundrect_rratio 0.25) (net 51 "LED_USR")))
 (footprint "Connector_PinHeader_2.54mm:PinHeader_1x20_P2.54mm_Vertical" (layer "F.Cu") (at 135.8 85)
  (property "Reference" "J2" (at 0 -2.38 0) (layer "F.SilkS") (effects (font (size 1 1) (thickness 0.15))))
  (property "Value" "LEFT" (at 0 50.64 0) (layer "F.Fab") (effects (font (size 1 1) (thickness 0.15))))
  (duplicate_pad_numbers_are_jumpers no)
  (pad "1" thru_hole rect (at 0 0) (size 1.7 1.7) (drill 1) (layers "*.Cu" "*.Mask") (remove_unused_layers no) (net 11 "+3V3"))
  (pad "2" thru_hole circle (at 0 2.54) (size 1.7 1.7) (drill 1) (layers "*.Cu" "*.Mask") (remove_unused_layers no) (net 13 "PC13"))
  (pad "3" thru_hole circle (at 0 5.08) (size 1.7 1.7) (drill 1) (layers "*.Cu" "*.Mask") (remove_unused_layers no) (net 14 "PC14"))
  (pad "4" thru_hole circle (at 0 7.62) (size 1.7 1.7) (drill 1) (layers "*.Cu" "*.Mask") (remove_unused_layers no) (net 15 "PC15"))
  (pad "5" thru_hole circle (at 0 10.16) (size 1.7 1.7) (drill 1) (layers "*.Cu" "*.Mask") (remove_unused_layers no) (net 19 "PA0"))
  (pad "6" thru_hole circle (at 0 12.7) (size 1.7 1.7) (drill 1) (layers "*.Cu" "*.Mask") (remove_unused_layers no) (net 20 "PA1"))
  (pad "7" thru_hole circle (at 0 15.24) (size 1.7 1.7) (drill 1) (layers "*.Cu" "*.Mask") (remove_unused_layers no) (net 21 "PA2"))
  (pad "8" thru_hole circle (at 0 17.78) (size 1.7 1.7) (drill 1) (layers "*.Cu" "*.Mask") (remove_unused_layers no) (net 22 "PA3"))
  (pad "9" thru_hole circle (at 0 20.32) (size 1.7 1.7) (drill 1) (layers "*.Cu" "*.Mask") (remove_unused_layers no) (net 23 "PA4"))
  (pad "10" thru_hole circle (at 0 22.86) (size 1.7 1.7) (drill 1) (layers "*.Cu" "*.Mask") (remove_unused_layers no) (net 24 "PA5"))
  (pad "11" thru_hole circle (at 0 25.4) (size 1.7 1.7) (drill 1) (layers "*.Cu" "*.Mask") (remove_unused_layers no) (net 25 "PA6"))
  (pad "12" thru_hole circle (at 0 27.94) (size 1.7 1.7) (drill 1) (layers "*.Cu" "*.Mask") (remove_unused_layers no) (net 26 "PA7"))
  (pad "13" thru_hole circle (at 0 30.48) (size 1.7 1.7) (drill 1) (layers "*.Cu" "*.Mask") (remove_unused_layers no) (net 27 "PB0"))
  (pad "14" thru_hole circle (at 0 33.02) (size 1.7 1.7) (drill 1) (layers "*.Cu" "*.Mask") (remove_unused_layers no) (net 28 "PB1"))
  (pad "15" thru_hole circle (at 0 35.56) (size 1.7 1.7) (drill 1) (layers "*.Cu" "*.Mask") (remove_unused_layers no) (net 30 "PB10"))
  (pad "16" thru_hole circle (at 0 38.1) (size 1.7 1.7) (drill 1) (layers "*.Cu" "*.Mask") (remove_unused_layers no) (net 31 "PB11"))
  (pad "17" thru_hole circle (at 0 40.64) (size 1.7 1.7) (drill 1) (layers "*.Cu" "*.Mask") (remove_unused_layers no) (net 18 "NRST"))
  (pad "18" thru_hole circle (at 0 43.18) (size 1.7 1.7) (drill 1) (layers "*.Cu" "*.Mask") (remove_unused_layers no) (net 11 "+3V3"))
  (pad "19" thru_hole circle (at 0 45.72) (size 1.7 1.7) (drill 1) (layers "*.Cu" "*.Mask") (remove_unused_layers no) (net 1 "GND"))
  (pad "20" thru_hole circle (at 0 48.26) (size 1.7 1.7) (drill 1) (layers "*.Cu" "*.Mask") (remove_unused_layers no) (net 1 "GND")))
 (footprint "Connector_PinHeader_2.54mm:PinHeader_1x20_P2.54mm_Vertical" (layer "F.Cu") (at 161.2 85)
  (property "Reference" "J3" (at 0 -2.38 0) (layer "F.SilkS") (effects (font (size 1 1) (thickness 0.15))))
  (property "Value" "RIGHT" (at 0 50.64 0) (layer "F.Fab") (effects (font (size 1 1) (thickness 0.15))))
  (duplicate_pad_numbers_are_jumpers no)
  (pad "1" thru_hole rect (at 0 0) (size 1.7 1.7) (drill 1) (layers "*.Cu" "*.Mask") (remove_unused_layers no) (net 11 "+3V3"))
  (pad "2" thru_hole circle (at 0 2.54) (size 1.7 1.7) (drill 1) (layers "*.Cu" "*.Mask") (remove_unused_layers no) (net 1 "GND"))
  (pad "3" thru_hole circle (at 0 5.08) (size 1.7 1.7) (drill 1) (layers "*.Cu" "*.Mask") (remove_unused_layers no) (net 2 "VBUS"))
  (pad "4" thru_hole circle (at 0 7.62) (size 1.7 1.7) (drill 1) (layers "*.Cu" "*.Mask") (remove_unused_layers no) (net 49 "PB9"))
  (pad "5" thru_hole circle (at 0 10.16) (size 1.7 1.7) (drill 1) (layers "*.Cu" "*.Mask") (remove_unused_layers no) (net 48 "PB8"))
  (pad "6" thru_hole circle (at 0 12.7) (size 1.7 1.7) (drill 1) (layers "*.Cu" "*.Mask") (remove_unused_layers no) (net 46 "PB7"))
  (pad "7" thru_hole circle (at 0 15.24) (size 1.7 1.7) (drill 1) (layers "*.Cu" "*.Mask") (remove_unused_layers no) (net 45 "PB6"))
  (pad "8" thru_hole circle (at 0 17.78) (size 1.7 1.7) (drill 1) (layers "*.Cu" "*.Mask") (remove_unused_layers no) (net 44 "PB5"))
  (pad "9" thru_hole circle (at 0 20.32) (size 1.7 1.7) (drill 1) (layers "*.Cu" "*.Mask") (remove_unused_layers no) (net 43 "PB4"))
  (pad "10" thru_hole circle (at 0 22.86) (size 1.7 1.7) (drill 1) (layers "*.Cu" "*.Mask") (remove_unused_layers no) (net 42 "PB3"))
  (pad "11" thru_hole circle (at 0 25.4) (size 1.7 1.7) (drill 1) (layers "*.Cu" "*.Mask") (remove_unused_layers no) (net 41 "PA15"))
  (pad "12" thru_hole circle (at 0 27.94) (size 1.7 1.7) (drill 1) (layers "*.Cu" "*.Mask") (remove_unused_layers no) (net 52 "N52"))
  (pad "13" thru_hole circle (at 0 30.48) (size 1.7 1.7) (drill 1) (layers "*.Cu" "*.Mask") (remove_unused_layers no) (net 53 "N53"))
  (pad "14" thru_hole circle (at 0 33.02) (size 1.7 1.7) (drill 1) (layers "*.Cu" "*.Mask") (remove_unused_layers no) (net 38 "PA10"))
  (pad "15" thru_hole circle (at 0 35.56) (size 1.7 1.7) (drill 1) (layers "*.Cu" "*.Mask") (remove_unused_layers no) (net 37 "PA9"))
  (pad "16" thru_hole circle (at 0 38.1) (size 1.7 1.7) (drill 1) (layers "*.Cu" "*.Mask") (remove_unused_layers no) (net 36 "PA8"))
  (pad "17" thru_hole circle (at 0 40.64) (size 1.7 1.7) (drill 1) (layers "*.Cu" "*.Mask") (remove_unused_layers no) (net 35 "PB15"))
  (pad "18" thru_hole circle (at 0 43.18) (size 1.7 1.7) (drill 1) (layers "*.Cu" "*.Mask") (remove_unused_layers no) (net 34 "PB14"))
  (pad "19" thru_hole circle (at 0 45.72) (size 1.7 1.7) (drill 1) (layers "*.Cu" "*.Mask") (remove_unused_layers no) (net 33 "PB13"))
  (pad "20" thru_hole circle (at 0 48.26) (size 1.7 1.7) (drill 1) (layers "*.Cu" "*.Mask") (remove_unused_layers no) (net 32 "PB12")))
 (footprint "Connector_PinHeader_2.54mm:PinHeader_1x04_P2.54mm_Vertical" (layer "F.Cu") (at 143.4 132 90)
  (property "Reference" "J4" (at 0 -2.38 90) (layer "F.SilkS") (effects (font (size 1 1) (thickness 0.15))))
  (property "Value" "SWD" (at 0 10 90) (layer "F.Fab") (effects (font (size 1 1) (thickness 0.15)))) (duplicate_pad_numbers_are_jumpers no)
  (pad "1" thru_hole rect (at 0 0 90) (size 1.7 1.7) (drill 1) (layers "*.Cu" "*.Mask") (remove_unused_layers no) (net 11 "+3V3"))
  (pad "2" thru_hole circle (at 0 2.54 90) (size 1.7 1.7) (drill 1) (layers "*.Cu" "*.Mask") (remove_unused_layers no) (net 39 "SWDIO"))
  (pad "3" thru_hole circle (at 0 5.08 90) (size 1.7 1.7) (drill 1) (layers "*.Cu" "*.Mask") (remove_unused_layers no) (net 40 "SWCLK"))
  (pad "4" thru_hole circle (at 0 7.62 90) (size 1.7 1.7) (drill 1) (layers "*.Cu" "*.Mask") (remove_unused_layers no) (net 1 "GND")))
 (via (at 147.95 82.0) (size 0.6) (drill 0.3) (layers "F.Cu" "B.Cu") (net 5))
 (via (at 149.4 84.75) (size 0.6) (drill 0.3) (layers "F.Cu" "B.Cu") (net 5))
 (via (at 150.6 83.4) (size 0.6) (drill 0.3) (layers "F.Cu" "B.Cu") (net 4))
 (via (at 154.2 84.75) (size 0.6) (drill 0.3) (layers "F.Cu" "B.Cu") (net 5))
 (via (at 155.7 106.3) (size 0.6) (drill 0.3) (layers "F.Cu" "B.Cu") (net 4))
 (via (at 155.7 107.7) (size 0.6) (drill 0.3) (layers "F.Cu" "B.Cu") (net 5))
 (segment (start 147.45 80.68) (end 147.4 81.5) (width 0.2) (layer "F.Cu") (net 4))
 (segment (start 147.4 81.5) (end 147.4 82.85) (width 0.2) (layer "F.Cu") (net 4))
 (segment (start 147.4 82.85) (end 148.337 82.85) (width 0.2) (layer "F.Cu") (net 4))
 (segment (start 146.45 80.68) (end 146.45 82.85) (width 0.2) (layer "F.Cu") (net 4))
 (segment (start 146.45 82.85) (end 146.063 82.85) (width 0.2) (layer "F.Cu") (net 4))
 (segment (start 146.95 80.68) (end 147.0 81.5) (width 0.2) (layer "F.Cu") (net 5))
 (segment (start 147.0 81.5) (end 147.0 84.75) (width 0.2) (layer "F.Cu") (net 5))
 (segment (start 147.0 84.75) (end 146.063 84.75) (width 0.2) (layer "F.Cu") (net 5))
 (segment (start 147.0 84.75) (end 148.337 84.75) (width 0.2) (layer "F.Cu") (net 5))
 (segment (start 147.95 80.68) (end 147.95 82.0) (width 0.2) (layer "F.Cu") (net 5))
 (segment (start 147.95 82.0) (end 149.4 83.45) (width 0.2) (layer "B.Cu") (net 5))
 (segment (start 149.4 83.45) (end 149.4 84.75) (width 0.2) (layer "B.Cu") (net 5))
 (segment (start 148.337 82.85) (end 150.05 82.85) (width 0.2) (layer "F.Cu") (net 4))
 (segment (start 150.05 82.85) (end 150.6 83.4) (width 0.2) (layer "F.Cu") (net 4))
 (segment (start 148.337 84.75) (end 149.4 84.75) (width 0.2) (layer "F.Cu") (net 5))
 (segment (start 149.4 84.75) (end 154.2 84.75) (width 0.2) (layer "F.Cu") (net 5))
 (segment (start 150.6 83.4) (end 151.8 83.4) (width 0.2) (layer "B.Cu") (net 4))
 (segment (start 151.8 83.4) (end 157.8 89.4) (width 0.2) (layer "B.Cu") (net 4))
 (segment (start 157.8 89.4) (end 157.8 104.2) (width 0.2) (layer "B.Cu") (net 4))
 (segment (start 157.8 104.2) (end 155.7 106.3) (width 0.2) (layer "B.Cu") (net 4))
 (segment (start 154.2 84.75) (end 158.5 89.05) (width 0.2) (layer "B.Cu") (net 5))
 (segment (start 158.5 89.05) (end 158.5 104.9) (width 0.2) (layer "B.Cu") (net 5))
 (segment (start 158.5 104.9) (end 155.7 107.7) (width 0.2) (layer "B.Cu") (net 5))
 (segment (start 155.7 106.3) (end 154.68 106.3) (width 0.2) (layer "F.Cu") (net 4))
 (segment (start 155.7 107.7) (end 154.68 107.7) (width 0.2) (layer "F.Cu") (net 5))
 (segment (start 151.862 106.75) (end 152.8 106.75) (width 0.2) (layer "F.Cu") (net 9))
 (segment (start 152.8 106.75) (end 153.25 106.3) (width 0.2) (layer "F.Cu") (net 9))
 (segment (start 153.25 106.3) (end 153.72 106.3) (width 0.2) (layer "F.Cu") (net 9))
 (segment (start 151.862 107.25) (end 152.8 107.25) (width 0.2) (layer "F.Cu") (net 10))
 (segment (start 152.8 107.25) (end 153.25 107.7) (width 0.2) (layer "F.Cu") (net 10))
 (segment (start 153.25 107.7) (end 153.72 107.7) (width 0.2) (layer "F.Cu") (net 10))
 (segment (start 153.72 105.38) (end 153.72 106.3) (width 0.2) (layer "F.Cu") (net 9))
 (segment (start 143.538 107.75) (end 142.1 107.75) (width 0.2) (layer "F.Cu") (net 17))
 (segment (start 142.1 107.75) (end 141.85 107.5) (width 0.2) (layer "F.Cu") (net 17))
 (segment (start 141.85 107.5) (end 139.5 107.5) (width 0.2) (layer "F.Cu") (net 17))
 (segment (start 139.5 107.5) (end 139.1 107.9) (width 0.2) (layer "F.Cu") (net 17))
 (segment (start 139.1 107.9) (end 138.7 108.35) (width 0.2) (layer "F.Cu") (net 17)))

